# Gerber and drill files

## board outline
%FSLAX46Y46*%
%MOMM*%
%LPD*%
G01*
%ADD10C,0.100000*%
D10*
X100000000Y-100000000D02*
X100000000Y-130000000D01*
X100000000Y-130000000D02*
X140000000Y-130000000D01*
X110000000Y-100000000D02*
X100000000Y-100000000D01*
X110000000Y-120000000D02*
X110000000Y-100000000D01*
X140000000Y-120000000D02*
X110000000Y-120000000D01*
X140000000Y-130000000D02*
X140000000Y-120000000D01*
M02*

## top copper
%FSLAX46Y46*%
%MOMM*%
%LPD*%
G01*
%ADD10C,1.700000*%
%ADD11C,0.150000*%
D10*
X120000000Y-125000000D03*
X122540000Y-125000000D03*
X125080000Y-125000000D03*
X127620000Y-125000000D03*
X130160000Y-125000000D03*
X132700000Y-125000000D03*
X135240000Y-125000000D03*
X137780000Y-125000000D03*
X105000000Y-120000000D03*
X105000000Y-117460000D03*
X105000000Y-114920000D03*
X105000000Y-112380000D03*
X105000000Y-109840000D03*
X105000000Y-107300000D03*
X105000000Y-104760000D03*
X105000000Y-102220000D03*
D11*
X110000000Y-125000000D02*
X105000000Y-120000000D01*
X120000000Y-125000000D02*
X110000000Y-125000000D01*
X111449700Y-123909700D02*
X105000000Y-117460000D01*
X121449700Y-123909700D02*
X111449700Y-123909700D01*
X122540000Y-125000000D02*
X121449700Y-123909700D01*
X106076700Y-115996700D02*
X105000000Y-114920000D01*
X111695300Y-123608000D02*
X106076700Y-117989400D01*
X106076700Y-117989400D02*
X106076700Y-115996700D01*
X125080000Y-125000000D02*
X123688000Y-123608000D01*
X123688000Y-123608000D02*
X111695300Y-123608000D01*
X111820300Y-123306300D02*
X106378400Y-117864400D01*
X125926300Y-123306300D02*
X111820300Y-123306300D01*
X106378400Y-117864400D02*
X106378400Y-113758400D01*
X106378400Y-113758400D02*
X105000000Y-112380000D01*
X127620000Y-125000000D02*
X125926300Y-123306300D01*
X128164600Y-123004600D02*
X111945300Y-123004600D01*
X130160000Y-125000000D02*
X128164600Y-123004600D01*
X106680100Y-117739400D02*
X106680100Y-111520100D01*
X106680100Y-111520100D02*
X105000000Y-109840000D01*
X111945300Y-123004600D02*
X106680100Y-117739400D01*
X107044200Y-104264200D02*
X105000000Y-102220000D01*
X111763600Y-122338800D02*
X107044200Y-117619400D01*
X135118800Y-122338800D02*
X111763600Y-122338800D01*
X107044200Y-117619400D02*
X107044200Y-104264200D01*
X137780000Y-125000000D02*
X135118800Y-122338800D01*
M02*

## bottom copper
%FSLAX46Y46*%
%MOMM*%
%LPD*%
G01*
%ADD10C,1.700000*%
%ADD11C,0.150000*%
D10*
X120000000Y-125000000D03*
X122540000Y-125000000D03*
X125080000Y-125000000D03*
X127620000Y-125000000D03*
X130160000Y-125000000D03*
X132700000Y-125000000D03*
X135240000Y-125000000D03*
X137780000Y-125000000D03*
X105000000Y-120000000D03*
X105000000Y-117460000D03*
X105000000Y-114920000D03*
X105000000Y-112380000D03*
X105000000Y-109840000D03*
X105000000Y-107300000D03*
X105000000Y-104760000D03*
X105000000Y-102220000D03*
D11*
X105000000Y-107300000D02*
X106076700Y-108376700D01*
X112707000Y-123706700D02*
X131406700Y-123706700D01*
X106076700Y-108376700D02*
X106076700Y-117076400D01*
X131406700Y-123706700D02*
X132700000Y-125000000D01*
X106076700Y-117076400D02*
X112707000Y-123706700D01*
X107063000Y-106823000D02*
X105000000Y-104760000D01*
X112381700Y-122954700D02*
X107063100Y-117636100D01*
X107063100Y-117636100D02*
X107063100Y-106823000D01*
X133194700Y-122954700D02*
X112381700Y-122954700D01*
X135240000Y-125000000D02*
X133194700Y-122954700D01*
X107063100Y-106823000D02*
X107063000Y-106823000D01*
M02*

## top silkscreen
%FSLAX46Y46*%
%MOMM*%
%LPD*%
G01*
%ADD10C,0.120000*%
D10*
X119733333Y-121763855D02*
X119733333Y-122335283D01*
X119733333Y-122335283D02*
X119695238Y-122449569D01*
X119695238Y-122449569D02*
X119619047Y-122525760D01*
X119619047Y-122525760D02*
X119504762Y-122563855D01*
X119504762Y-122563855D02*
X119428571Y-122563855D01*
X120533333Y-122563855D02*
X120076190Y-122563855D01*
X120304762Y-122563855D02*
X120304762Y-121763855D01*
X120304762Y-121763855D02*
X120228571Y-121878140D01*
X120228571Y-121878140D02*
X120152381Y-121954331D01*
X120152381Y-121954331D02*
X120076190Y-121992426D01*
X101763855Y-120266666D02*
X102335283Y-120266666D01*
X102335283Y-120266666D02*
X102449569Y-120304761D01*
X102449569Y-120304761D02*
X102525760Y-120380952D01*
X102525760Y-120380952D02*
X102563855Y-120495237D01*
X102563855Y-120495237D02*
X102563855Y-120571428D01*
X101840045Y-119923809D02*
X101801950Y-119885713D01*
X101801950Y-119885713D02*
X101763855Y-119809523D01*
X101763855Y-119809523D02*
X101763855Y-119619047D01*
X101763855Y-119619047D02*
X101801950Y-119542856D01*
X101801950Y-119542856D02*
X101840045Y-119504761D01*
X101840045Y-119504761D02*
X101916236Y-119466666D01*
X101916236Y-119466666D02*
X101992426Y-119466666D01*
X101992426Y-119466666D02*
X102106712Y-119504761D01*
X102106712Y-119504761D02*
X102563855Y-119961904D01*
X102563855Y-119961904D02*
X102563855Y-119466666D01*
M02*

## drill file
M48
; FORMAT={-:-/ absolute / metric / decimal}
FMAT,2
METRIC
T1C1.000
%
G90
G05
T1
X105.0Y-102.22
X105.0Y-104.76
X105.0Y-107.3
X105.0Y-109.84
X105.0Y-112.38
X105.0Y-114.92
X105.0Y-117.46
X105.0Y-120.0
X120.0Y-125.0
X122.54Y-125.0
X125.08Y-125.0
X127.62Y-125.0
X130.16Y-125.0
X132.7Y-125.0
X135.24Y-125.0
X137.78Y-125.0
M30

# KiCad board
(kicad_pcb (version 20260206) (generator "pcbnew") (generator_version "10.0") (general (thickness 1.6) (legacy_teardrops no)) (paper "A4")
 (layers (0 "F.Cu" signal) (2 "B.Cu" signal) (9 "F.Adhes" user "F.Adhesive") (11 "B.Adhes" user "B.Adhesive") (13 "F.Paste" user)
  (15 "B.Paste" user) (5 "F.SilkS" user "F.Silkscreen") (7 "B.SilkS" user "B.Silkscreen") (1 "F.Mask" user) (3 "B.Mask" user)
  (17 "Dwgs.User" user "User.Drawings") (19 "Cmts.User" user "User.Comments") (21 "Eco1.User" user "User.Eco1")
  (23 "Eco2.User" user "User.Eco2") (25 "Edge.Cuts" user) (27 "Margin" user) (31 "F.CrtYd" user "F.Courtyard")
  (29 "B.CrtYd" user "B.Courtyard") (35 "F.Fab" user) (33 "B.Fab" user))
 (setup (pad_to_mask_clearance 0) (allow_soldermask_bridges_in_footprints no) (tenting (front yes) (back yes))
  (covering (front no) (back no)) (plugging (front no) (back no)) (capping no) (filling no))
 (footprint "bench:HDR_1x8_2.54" (layer "F.Cu") (at 120 125)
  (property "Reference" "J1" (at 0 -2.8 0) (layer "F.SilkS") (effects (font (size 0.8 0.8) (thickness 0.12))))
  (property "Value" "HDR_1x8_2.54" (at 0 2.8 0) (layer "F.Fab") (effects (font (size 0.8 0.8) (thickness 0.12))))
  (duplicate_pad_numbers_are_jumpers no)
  (pad "1" thru_hole circle (at 0 0) (size 1.7 1.7) (drill 1) (layers "*.Cu" "*.Mask") (remove_unused_layers no) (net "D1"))
  (pad "2" thru_hole circle (at 2.54 0) (size 1.7 1.7) (drill 1) (layers "*.Cu" "*.Mask") (remove_unused_layers no) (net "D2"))
  (pad "3" thru_hole circle (at 5.08 0) (size 1.7 1.7) (drill 1) (layers "*.Cu" "*.Mask") (remove_unused_layers no) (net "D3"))
  (pad "4" thru_hole circle (at 7.62 0) (size 1.7 1.7) (drill 1) (layers "*.Cu" "*.Mask") (remove_unused_layers no) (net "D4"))
  (pad "5" thru_hole circle (at 10.16 0) (size 1.7 1.7) (drill 1) (layers "*.Cu" "*.Mask") (remove_unused_layers no) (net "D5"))
  (pad "6" thru_hole circle (at 12.7 0) (size 1.7 1.7) (drill 1) (layers "*.Cu" "*.Mask") (remove_unused_layers no) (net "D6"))
  (pad "7" thru_hole circle (at 15.24 0) (size 1.7 1.7) (drill 1) (layers "*.Cu" "*.Mask") (remove_unused_layers no) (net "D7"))
  (pad "8" thru_hole circle (at 17.78 0) (size 1.7 1.7) (drill 1) (layers "*.Cu" "*.Mask") (remove_unused_layers no) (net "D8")))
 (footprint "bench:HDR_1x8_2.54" (layer "F.Cu") (at 105 120 90)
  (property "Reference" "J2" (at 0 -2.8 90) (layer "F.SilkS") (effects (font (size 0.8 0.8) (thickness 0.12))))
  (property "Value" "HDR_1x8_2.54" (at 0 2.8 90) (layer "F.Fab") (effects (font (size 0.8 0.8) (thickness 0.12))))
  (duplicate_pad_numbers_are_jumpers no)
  (pad "1" thru_hole circle (at 0 0 90) (size 1.7 1.7) (drill 1) (layers "*.Cu" "*.Mask") (remove_unused_layers no) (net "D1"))
  (pad "2" thru_hole circle (at 2.54 0 90) (size 1.7 1.7) (drill 1) (layers "*.Cu" "*.Mask") (remove_unused_layers no) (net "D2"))
  (pad "3" thru_hole circle (at 5.08 0 90) (size 1.7 1.7) (drill 1) (layers "*.Cu" "*.Mask") (remove_unused_layers no) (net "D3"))
  (pad "4" thru_hole circle (at 7.62 0 90) (size 1.7 1.7) (drill 1) (layers "*.Cu" "*.Mask") (remove_unused_layers no) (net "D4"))
  (pad "5" thru_hole circle (at 10.16 0 90) (size 1.7 1.7) (drill 1) (layers "*.Cu" "*.Mask") (remove_unused_layers no) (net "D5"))
  (pad "6" thru_hole circle (at 12.7 0 90) (size 1.7 1.7) (drill 1) (layers "*.Cu" "*.Mask") (remove_unused_layers no) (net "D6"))
  (pad "7" thru_hole circle (at 15.24 0 90) (size 1.7 1.7) (drill 1) (layers "*.Cu" "*.Mask") (remove_unused_layers no) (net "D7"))
  (pad "8" thru_hole circle (at 17.78 0 90) (size 1.7 1.7) (drill 1) (layers "*.Cu" "*.Mask") (remove_unused_layers no) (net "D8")))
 (gr_line (start 100 100) (end 100 130) (stroke (width 0.1) (type solid)) (layer "Edge.Cuts"))
 (gr_line (start 100 130) (end 140 130) (stroke (width 0.1) (type solid)) (layer "Edge.Cuts"))
 (gr_line (start 110 100) (end 100 100) (stroke (width 0.1) (type solid)) (layer "Edge.Cuts"))
 (gr_line (start 110 120) (end 110 100) (stroke (width 0.1) (type solid)) (layer "Edge.Cuts"))
 (gr_line (start 140 120) (end 110 120) (stroke (width 0.1) (type solid)) (layer "Edge.Cuts"))
 (gr_line (start 140 130) (end 140 120) (stroke (width 0.1) (type solid)) (layer "Edge.Cuts"))
 (segment (start 110 125) (end 105 120) (width 0.15) (layer "F.Cu") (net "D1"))
 (segment (start 120 125) (end 110 125) (width 0.15) (layer "F.Cu") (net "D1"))
 (segment (start 111.4497 123.9097) (end 105 117.46) (width 0.15) (layer "F.Cu") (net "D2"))
 (segment (start 121.4497 123.9097) (end 111.4497 123.9097) (width 0.15) (layer "F.Cu") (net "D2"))
 (segment (start 122.54 125) (end 121.4497 123.9097) (width 0.15) (layer "F.Cu") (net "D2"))
 (segment (start 106.0767 115.9967) (end 105 114.92) (width 0.15) (layer "F.Cu") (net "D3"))
 (segment (start 111.6953 123.608) (end 106.0767 117.9894) (width 0.15) (layer "F.Cu") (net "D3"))
 (segment (start 106.0767 117.9894) (end 106.0767 115.9967) (width 0.15) (layer "F.Cu") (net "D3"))
 (segment (start 125.08 125) (end 123.688 123.608) (width 0.15) (layer "F.Cu") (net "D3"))
 (segment (start 123.688 123.608) (end 111.6953 123.608) (width 0.15) (layer "F.Cu") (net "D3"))
 (segment (start 111.8203 123.3063) (end 106.3784 117.8644) (width 0.15) (layer "F.Cu") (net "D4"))
 (segment (start 125.9263 123.3063) (end 111.8203 123.3063) (width 0.15) (layer "F.Cu") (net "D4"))
 (segment (start 106.3784 117.8644) (end 106.3784 113.7584) (width 0.15) (layer "F.Cu") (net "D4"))
 (segment (start 106.3784 113.7584) (end 105 112.38) (width 0.15) (layer "F.Cu") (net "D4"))
 (segment (start 127.62 125) (end 125.9263 123.3063) (width 0.15) (layer "F.Cu") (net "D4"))
 (segment (start 128.1646 123.0046) (end 111.9453 123.0046) (width 0.15) (layer "F.Cu") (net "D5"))
 (segment (start 130.16 125) (end 128.1646 123.0046) (width 0.15) (layer "F.Cu") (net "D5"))
 (segment (start 106.6801 117.7394) (end 106.6801 111.5201) (width 0.15) (layer "F.Cu") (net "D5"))
 (segment (start 106.6801 111.5201) (end 105 109.84) (width 0.15) (layer "F.Cu") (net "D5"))
 (segment (start 111.9453 123.0046) (end 106.6801 117.7394) (width 0.15) (layer "F.Cu") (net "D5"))
 (segment (start 105 107.3) (end 106.0767 108.3767) (width 0.15) (layer "B.Cu") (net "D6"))
 (segment (start 112.707 123.7067) (end 131.4067 123.7067) (width 0.15) (layer "B.Cu") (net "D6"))
 (segment (start 106.0767 108.3767) (end 106.0767 117.0764) (width 0.15) (layer "B.Cu") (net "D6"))
 (segment (start 131.4067 123.7067) (end 132.7 125) (width 0.15) (layer "B.Cu") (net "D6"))
 (segment (start 106.0767 117.0764) (end 112.707 123.7067) (width 0.15) (layer "B.Cu") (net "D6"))
 (segment (start 107.063 106.823) (end 105 104.76) (width 0.15) (layer "B.Cu") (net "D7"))
 (segment (start 112.3817 122.9547) (end 107.0631 117.6361) (width 0.15) (layer "B.Cu") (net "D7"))
 (segment (start 107.0631 117.6361) (end 107.0631 106.823) (width 0.15) (layer "B.Cu") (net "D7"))
 (segment (start 133.1947 122.9547) (end 112.3817 122.9547) (width 0.15) (layer "B.Cu") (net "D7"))
 (segment (start 135.24 125) (end 133.1947 122.9547) (width 0.15) (layer "B.Cu") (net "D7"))
 (segment (start 107.0631 106.823) (end 107.063 106.823) (width 0.15) (layer "B.Cu") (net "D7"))
 (segment (start 107.0442 104.2642) (end 105 102.22) (width 0.15) (layer "F.Cu") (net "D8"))
 (segment (start 111.7636 122.3388) (end 107.0442 117.6194) (width 0.15) (layer "F.Cu") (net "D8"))
 (segment (start 135.1188 122.3388) (end 111.7636 122.3388) (width 0.15) (layer "F.Cu") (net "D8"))
 (segment (start 107.0442 117.6194) (end 107.0442 104.2642) (width 0.15) (layer "F.Cu") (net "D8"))
 (segment (start 137.78 125) (end 135.1188 122.3388) (width 0.15) (layer "F.Cu") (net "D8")))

